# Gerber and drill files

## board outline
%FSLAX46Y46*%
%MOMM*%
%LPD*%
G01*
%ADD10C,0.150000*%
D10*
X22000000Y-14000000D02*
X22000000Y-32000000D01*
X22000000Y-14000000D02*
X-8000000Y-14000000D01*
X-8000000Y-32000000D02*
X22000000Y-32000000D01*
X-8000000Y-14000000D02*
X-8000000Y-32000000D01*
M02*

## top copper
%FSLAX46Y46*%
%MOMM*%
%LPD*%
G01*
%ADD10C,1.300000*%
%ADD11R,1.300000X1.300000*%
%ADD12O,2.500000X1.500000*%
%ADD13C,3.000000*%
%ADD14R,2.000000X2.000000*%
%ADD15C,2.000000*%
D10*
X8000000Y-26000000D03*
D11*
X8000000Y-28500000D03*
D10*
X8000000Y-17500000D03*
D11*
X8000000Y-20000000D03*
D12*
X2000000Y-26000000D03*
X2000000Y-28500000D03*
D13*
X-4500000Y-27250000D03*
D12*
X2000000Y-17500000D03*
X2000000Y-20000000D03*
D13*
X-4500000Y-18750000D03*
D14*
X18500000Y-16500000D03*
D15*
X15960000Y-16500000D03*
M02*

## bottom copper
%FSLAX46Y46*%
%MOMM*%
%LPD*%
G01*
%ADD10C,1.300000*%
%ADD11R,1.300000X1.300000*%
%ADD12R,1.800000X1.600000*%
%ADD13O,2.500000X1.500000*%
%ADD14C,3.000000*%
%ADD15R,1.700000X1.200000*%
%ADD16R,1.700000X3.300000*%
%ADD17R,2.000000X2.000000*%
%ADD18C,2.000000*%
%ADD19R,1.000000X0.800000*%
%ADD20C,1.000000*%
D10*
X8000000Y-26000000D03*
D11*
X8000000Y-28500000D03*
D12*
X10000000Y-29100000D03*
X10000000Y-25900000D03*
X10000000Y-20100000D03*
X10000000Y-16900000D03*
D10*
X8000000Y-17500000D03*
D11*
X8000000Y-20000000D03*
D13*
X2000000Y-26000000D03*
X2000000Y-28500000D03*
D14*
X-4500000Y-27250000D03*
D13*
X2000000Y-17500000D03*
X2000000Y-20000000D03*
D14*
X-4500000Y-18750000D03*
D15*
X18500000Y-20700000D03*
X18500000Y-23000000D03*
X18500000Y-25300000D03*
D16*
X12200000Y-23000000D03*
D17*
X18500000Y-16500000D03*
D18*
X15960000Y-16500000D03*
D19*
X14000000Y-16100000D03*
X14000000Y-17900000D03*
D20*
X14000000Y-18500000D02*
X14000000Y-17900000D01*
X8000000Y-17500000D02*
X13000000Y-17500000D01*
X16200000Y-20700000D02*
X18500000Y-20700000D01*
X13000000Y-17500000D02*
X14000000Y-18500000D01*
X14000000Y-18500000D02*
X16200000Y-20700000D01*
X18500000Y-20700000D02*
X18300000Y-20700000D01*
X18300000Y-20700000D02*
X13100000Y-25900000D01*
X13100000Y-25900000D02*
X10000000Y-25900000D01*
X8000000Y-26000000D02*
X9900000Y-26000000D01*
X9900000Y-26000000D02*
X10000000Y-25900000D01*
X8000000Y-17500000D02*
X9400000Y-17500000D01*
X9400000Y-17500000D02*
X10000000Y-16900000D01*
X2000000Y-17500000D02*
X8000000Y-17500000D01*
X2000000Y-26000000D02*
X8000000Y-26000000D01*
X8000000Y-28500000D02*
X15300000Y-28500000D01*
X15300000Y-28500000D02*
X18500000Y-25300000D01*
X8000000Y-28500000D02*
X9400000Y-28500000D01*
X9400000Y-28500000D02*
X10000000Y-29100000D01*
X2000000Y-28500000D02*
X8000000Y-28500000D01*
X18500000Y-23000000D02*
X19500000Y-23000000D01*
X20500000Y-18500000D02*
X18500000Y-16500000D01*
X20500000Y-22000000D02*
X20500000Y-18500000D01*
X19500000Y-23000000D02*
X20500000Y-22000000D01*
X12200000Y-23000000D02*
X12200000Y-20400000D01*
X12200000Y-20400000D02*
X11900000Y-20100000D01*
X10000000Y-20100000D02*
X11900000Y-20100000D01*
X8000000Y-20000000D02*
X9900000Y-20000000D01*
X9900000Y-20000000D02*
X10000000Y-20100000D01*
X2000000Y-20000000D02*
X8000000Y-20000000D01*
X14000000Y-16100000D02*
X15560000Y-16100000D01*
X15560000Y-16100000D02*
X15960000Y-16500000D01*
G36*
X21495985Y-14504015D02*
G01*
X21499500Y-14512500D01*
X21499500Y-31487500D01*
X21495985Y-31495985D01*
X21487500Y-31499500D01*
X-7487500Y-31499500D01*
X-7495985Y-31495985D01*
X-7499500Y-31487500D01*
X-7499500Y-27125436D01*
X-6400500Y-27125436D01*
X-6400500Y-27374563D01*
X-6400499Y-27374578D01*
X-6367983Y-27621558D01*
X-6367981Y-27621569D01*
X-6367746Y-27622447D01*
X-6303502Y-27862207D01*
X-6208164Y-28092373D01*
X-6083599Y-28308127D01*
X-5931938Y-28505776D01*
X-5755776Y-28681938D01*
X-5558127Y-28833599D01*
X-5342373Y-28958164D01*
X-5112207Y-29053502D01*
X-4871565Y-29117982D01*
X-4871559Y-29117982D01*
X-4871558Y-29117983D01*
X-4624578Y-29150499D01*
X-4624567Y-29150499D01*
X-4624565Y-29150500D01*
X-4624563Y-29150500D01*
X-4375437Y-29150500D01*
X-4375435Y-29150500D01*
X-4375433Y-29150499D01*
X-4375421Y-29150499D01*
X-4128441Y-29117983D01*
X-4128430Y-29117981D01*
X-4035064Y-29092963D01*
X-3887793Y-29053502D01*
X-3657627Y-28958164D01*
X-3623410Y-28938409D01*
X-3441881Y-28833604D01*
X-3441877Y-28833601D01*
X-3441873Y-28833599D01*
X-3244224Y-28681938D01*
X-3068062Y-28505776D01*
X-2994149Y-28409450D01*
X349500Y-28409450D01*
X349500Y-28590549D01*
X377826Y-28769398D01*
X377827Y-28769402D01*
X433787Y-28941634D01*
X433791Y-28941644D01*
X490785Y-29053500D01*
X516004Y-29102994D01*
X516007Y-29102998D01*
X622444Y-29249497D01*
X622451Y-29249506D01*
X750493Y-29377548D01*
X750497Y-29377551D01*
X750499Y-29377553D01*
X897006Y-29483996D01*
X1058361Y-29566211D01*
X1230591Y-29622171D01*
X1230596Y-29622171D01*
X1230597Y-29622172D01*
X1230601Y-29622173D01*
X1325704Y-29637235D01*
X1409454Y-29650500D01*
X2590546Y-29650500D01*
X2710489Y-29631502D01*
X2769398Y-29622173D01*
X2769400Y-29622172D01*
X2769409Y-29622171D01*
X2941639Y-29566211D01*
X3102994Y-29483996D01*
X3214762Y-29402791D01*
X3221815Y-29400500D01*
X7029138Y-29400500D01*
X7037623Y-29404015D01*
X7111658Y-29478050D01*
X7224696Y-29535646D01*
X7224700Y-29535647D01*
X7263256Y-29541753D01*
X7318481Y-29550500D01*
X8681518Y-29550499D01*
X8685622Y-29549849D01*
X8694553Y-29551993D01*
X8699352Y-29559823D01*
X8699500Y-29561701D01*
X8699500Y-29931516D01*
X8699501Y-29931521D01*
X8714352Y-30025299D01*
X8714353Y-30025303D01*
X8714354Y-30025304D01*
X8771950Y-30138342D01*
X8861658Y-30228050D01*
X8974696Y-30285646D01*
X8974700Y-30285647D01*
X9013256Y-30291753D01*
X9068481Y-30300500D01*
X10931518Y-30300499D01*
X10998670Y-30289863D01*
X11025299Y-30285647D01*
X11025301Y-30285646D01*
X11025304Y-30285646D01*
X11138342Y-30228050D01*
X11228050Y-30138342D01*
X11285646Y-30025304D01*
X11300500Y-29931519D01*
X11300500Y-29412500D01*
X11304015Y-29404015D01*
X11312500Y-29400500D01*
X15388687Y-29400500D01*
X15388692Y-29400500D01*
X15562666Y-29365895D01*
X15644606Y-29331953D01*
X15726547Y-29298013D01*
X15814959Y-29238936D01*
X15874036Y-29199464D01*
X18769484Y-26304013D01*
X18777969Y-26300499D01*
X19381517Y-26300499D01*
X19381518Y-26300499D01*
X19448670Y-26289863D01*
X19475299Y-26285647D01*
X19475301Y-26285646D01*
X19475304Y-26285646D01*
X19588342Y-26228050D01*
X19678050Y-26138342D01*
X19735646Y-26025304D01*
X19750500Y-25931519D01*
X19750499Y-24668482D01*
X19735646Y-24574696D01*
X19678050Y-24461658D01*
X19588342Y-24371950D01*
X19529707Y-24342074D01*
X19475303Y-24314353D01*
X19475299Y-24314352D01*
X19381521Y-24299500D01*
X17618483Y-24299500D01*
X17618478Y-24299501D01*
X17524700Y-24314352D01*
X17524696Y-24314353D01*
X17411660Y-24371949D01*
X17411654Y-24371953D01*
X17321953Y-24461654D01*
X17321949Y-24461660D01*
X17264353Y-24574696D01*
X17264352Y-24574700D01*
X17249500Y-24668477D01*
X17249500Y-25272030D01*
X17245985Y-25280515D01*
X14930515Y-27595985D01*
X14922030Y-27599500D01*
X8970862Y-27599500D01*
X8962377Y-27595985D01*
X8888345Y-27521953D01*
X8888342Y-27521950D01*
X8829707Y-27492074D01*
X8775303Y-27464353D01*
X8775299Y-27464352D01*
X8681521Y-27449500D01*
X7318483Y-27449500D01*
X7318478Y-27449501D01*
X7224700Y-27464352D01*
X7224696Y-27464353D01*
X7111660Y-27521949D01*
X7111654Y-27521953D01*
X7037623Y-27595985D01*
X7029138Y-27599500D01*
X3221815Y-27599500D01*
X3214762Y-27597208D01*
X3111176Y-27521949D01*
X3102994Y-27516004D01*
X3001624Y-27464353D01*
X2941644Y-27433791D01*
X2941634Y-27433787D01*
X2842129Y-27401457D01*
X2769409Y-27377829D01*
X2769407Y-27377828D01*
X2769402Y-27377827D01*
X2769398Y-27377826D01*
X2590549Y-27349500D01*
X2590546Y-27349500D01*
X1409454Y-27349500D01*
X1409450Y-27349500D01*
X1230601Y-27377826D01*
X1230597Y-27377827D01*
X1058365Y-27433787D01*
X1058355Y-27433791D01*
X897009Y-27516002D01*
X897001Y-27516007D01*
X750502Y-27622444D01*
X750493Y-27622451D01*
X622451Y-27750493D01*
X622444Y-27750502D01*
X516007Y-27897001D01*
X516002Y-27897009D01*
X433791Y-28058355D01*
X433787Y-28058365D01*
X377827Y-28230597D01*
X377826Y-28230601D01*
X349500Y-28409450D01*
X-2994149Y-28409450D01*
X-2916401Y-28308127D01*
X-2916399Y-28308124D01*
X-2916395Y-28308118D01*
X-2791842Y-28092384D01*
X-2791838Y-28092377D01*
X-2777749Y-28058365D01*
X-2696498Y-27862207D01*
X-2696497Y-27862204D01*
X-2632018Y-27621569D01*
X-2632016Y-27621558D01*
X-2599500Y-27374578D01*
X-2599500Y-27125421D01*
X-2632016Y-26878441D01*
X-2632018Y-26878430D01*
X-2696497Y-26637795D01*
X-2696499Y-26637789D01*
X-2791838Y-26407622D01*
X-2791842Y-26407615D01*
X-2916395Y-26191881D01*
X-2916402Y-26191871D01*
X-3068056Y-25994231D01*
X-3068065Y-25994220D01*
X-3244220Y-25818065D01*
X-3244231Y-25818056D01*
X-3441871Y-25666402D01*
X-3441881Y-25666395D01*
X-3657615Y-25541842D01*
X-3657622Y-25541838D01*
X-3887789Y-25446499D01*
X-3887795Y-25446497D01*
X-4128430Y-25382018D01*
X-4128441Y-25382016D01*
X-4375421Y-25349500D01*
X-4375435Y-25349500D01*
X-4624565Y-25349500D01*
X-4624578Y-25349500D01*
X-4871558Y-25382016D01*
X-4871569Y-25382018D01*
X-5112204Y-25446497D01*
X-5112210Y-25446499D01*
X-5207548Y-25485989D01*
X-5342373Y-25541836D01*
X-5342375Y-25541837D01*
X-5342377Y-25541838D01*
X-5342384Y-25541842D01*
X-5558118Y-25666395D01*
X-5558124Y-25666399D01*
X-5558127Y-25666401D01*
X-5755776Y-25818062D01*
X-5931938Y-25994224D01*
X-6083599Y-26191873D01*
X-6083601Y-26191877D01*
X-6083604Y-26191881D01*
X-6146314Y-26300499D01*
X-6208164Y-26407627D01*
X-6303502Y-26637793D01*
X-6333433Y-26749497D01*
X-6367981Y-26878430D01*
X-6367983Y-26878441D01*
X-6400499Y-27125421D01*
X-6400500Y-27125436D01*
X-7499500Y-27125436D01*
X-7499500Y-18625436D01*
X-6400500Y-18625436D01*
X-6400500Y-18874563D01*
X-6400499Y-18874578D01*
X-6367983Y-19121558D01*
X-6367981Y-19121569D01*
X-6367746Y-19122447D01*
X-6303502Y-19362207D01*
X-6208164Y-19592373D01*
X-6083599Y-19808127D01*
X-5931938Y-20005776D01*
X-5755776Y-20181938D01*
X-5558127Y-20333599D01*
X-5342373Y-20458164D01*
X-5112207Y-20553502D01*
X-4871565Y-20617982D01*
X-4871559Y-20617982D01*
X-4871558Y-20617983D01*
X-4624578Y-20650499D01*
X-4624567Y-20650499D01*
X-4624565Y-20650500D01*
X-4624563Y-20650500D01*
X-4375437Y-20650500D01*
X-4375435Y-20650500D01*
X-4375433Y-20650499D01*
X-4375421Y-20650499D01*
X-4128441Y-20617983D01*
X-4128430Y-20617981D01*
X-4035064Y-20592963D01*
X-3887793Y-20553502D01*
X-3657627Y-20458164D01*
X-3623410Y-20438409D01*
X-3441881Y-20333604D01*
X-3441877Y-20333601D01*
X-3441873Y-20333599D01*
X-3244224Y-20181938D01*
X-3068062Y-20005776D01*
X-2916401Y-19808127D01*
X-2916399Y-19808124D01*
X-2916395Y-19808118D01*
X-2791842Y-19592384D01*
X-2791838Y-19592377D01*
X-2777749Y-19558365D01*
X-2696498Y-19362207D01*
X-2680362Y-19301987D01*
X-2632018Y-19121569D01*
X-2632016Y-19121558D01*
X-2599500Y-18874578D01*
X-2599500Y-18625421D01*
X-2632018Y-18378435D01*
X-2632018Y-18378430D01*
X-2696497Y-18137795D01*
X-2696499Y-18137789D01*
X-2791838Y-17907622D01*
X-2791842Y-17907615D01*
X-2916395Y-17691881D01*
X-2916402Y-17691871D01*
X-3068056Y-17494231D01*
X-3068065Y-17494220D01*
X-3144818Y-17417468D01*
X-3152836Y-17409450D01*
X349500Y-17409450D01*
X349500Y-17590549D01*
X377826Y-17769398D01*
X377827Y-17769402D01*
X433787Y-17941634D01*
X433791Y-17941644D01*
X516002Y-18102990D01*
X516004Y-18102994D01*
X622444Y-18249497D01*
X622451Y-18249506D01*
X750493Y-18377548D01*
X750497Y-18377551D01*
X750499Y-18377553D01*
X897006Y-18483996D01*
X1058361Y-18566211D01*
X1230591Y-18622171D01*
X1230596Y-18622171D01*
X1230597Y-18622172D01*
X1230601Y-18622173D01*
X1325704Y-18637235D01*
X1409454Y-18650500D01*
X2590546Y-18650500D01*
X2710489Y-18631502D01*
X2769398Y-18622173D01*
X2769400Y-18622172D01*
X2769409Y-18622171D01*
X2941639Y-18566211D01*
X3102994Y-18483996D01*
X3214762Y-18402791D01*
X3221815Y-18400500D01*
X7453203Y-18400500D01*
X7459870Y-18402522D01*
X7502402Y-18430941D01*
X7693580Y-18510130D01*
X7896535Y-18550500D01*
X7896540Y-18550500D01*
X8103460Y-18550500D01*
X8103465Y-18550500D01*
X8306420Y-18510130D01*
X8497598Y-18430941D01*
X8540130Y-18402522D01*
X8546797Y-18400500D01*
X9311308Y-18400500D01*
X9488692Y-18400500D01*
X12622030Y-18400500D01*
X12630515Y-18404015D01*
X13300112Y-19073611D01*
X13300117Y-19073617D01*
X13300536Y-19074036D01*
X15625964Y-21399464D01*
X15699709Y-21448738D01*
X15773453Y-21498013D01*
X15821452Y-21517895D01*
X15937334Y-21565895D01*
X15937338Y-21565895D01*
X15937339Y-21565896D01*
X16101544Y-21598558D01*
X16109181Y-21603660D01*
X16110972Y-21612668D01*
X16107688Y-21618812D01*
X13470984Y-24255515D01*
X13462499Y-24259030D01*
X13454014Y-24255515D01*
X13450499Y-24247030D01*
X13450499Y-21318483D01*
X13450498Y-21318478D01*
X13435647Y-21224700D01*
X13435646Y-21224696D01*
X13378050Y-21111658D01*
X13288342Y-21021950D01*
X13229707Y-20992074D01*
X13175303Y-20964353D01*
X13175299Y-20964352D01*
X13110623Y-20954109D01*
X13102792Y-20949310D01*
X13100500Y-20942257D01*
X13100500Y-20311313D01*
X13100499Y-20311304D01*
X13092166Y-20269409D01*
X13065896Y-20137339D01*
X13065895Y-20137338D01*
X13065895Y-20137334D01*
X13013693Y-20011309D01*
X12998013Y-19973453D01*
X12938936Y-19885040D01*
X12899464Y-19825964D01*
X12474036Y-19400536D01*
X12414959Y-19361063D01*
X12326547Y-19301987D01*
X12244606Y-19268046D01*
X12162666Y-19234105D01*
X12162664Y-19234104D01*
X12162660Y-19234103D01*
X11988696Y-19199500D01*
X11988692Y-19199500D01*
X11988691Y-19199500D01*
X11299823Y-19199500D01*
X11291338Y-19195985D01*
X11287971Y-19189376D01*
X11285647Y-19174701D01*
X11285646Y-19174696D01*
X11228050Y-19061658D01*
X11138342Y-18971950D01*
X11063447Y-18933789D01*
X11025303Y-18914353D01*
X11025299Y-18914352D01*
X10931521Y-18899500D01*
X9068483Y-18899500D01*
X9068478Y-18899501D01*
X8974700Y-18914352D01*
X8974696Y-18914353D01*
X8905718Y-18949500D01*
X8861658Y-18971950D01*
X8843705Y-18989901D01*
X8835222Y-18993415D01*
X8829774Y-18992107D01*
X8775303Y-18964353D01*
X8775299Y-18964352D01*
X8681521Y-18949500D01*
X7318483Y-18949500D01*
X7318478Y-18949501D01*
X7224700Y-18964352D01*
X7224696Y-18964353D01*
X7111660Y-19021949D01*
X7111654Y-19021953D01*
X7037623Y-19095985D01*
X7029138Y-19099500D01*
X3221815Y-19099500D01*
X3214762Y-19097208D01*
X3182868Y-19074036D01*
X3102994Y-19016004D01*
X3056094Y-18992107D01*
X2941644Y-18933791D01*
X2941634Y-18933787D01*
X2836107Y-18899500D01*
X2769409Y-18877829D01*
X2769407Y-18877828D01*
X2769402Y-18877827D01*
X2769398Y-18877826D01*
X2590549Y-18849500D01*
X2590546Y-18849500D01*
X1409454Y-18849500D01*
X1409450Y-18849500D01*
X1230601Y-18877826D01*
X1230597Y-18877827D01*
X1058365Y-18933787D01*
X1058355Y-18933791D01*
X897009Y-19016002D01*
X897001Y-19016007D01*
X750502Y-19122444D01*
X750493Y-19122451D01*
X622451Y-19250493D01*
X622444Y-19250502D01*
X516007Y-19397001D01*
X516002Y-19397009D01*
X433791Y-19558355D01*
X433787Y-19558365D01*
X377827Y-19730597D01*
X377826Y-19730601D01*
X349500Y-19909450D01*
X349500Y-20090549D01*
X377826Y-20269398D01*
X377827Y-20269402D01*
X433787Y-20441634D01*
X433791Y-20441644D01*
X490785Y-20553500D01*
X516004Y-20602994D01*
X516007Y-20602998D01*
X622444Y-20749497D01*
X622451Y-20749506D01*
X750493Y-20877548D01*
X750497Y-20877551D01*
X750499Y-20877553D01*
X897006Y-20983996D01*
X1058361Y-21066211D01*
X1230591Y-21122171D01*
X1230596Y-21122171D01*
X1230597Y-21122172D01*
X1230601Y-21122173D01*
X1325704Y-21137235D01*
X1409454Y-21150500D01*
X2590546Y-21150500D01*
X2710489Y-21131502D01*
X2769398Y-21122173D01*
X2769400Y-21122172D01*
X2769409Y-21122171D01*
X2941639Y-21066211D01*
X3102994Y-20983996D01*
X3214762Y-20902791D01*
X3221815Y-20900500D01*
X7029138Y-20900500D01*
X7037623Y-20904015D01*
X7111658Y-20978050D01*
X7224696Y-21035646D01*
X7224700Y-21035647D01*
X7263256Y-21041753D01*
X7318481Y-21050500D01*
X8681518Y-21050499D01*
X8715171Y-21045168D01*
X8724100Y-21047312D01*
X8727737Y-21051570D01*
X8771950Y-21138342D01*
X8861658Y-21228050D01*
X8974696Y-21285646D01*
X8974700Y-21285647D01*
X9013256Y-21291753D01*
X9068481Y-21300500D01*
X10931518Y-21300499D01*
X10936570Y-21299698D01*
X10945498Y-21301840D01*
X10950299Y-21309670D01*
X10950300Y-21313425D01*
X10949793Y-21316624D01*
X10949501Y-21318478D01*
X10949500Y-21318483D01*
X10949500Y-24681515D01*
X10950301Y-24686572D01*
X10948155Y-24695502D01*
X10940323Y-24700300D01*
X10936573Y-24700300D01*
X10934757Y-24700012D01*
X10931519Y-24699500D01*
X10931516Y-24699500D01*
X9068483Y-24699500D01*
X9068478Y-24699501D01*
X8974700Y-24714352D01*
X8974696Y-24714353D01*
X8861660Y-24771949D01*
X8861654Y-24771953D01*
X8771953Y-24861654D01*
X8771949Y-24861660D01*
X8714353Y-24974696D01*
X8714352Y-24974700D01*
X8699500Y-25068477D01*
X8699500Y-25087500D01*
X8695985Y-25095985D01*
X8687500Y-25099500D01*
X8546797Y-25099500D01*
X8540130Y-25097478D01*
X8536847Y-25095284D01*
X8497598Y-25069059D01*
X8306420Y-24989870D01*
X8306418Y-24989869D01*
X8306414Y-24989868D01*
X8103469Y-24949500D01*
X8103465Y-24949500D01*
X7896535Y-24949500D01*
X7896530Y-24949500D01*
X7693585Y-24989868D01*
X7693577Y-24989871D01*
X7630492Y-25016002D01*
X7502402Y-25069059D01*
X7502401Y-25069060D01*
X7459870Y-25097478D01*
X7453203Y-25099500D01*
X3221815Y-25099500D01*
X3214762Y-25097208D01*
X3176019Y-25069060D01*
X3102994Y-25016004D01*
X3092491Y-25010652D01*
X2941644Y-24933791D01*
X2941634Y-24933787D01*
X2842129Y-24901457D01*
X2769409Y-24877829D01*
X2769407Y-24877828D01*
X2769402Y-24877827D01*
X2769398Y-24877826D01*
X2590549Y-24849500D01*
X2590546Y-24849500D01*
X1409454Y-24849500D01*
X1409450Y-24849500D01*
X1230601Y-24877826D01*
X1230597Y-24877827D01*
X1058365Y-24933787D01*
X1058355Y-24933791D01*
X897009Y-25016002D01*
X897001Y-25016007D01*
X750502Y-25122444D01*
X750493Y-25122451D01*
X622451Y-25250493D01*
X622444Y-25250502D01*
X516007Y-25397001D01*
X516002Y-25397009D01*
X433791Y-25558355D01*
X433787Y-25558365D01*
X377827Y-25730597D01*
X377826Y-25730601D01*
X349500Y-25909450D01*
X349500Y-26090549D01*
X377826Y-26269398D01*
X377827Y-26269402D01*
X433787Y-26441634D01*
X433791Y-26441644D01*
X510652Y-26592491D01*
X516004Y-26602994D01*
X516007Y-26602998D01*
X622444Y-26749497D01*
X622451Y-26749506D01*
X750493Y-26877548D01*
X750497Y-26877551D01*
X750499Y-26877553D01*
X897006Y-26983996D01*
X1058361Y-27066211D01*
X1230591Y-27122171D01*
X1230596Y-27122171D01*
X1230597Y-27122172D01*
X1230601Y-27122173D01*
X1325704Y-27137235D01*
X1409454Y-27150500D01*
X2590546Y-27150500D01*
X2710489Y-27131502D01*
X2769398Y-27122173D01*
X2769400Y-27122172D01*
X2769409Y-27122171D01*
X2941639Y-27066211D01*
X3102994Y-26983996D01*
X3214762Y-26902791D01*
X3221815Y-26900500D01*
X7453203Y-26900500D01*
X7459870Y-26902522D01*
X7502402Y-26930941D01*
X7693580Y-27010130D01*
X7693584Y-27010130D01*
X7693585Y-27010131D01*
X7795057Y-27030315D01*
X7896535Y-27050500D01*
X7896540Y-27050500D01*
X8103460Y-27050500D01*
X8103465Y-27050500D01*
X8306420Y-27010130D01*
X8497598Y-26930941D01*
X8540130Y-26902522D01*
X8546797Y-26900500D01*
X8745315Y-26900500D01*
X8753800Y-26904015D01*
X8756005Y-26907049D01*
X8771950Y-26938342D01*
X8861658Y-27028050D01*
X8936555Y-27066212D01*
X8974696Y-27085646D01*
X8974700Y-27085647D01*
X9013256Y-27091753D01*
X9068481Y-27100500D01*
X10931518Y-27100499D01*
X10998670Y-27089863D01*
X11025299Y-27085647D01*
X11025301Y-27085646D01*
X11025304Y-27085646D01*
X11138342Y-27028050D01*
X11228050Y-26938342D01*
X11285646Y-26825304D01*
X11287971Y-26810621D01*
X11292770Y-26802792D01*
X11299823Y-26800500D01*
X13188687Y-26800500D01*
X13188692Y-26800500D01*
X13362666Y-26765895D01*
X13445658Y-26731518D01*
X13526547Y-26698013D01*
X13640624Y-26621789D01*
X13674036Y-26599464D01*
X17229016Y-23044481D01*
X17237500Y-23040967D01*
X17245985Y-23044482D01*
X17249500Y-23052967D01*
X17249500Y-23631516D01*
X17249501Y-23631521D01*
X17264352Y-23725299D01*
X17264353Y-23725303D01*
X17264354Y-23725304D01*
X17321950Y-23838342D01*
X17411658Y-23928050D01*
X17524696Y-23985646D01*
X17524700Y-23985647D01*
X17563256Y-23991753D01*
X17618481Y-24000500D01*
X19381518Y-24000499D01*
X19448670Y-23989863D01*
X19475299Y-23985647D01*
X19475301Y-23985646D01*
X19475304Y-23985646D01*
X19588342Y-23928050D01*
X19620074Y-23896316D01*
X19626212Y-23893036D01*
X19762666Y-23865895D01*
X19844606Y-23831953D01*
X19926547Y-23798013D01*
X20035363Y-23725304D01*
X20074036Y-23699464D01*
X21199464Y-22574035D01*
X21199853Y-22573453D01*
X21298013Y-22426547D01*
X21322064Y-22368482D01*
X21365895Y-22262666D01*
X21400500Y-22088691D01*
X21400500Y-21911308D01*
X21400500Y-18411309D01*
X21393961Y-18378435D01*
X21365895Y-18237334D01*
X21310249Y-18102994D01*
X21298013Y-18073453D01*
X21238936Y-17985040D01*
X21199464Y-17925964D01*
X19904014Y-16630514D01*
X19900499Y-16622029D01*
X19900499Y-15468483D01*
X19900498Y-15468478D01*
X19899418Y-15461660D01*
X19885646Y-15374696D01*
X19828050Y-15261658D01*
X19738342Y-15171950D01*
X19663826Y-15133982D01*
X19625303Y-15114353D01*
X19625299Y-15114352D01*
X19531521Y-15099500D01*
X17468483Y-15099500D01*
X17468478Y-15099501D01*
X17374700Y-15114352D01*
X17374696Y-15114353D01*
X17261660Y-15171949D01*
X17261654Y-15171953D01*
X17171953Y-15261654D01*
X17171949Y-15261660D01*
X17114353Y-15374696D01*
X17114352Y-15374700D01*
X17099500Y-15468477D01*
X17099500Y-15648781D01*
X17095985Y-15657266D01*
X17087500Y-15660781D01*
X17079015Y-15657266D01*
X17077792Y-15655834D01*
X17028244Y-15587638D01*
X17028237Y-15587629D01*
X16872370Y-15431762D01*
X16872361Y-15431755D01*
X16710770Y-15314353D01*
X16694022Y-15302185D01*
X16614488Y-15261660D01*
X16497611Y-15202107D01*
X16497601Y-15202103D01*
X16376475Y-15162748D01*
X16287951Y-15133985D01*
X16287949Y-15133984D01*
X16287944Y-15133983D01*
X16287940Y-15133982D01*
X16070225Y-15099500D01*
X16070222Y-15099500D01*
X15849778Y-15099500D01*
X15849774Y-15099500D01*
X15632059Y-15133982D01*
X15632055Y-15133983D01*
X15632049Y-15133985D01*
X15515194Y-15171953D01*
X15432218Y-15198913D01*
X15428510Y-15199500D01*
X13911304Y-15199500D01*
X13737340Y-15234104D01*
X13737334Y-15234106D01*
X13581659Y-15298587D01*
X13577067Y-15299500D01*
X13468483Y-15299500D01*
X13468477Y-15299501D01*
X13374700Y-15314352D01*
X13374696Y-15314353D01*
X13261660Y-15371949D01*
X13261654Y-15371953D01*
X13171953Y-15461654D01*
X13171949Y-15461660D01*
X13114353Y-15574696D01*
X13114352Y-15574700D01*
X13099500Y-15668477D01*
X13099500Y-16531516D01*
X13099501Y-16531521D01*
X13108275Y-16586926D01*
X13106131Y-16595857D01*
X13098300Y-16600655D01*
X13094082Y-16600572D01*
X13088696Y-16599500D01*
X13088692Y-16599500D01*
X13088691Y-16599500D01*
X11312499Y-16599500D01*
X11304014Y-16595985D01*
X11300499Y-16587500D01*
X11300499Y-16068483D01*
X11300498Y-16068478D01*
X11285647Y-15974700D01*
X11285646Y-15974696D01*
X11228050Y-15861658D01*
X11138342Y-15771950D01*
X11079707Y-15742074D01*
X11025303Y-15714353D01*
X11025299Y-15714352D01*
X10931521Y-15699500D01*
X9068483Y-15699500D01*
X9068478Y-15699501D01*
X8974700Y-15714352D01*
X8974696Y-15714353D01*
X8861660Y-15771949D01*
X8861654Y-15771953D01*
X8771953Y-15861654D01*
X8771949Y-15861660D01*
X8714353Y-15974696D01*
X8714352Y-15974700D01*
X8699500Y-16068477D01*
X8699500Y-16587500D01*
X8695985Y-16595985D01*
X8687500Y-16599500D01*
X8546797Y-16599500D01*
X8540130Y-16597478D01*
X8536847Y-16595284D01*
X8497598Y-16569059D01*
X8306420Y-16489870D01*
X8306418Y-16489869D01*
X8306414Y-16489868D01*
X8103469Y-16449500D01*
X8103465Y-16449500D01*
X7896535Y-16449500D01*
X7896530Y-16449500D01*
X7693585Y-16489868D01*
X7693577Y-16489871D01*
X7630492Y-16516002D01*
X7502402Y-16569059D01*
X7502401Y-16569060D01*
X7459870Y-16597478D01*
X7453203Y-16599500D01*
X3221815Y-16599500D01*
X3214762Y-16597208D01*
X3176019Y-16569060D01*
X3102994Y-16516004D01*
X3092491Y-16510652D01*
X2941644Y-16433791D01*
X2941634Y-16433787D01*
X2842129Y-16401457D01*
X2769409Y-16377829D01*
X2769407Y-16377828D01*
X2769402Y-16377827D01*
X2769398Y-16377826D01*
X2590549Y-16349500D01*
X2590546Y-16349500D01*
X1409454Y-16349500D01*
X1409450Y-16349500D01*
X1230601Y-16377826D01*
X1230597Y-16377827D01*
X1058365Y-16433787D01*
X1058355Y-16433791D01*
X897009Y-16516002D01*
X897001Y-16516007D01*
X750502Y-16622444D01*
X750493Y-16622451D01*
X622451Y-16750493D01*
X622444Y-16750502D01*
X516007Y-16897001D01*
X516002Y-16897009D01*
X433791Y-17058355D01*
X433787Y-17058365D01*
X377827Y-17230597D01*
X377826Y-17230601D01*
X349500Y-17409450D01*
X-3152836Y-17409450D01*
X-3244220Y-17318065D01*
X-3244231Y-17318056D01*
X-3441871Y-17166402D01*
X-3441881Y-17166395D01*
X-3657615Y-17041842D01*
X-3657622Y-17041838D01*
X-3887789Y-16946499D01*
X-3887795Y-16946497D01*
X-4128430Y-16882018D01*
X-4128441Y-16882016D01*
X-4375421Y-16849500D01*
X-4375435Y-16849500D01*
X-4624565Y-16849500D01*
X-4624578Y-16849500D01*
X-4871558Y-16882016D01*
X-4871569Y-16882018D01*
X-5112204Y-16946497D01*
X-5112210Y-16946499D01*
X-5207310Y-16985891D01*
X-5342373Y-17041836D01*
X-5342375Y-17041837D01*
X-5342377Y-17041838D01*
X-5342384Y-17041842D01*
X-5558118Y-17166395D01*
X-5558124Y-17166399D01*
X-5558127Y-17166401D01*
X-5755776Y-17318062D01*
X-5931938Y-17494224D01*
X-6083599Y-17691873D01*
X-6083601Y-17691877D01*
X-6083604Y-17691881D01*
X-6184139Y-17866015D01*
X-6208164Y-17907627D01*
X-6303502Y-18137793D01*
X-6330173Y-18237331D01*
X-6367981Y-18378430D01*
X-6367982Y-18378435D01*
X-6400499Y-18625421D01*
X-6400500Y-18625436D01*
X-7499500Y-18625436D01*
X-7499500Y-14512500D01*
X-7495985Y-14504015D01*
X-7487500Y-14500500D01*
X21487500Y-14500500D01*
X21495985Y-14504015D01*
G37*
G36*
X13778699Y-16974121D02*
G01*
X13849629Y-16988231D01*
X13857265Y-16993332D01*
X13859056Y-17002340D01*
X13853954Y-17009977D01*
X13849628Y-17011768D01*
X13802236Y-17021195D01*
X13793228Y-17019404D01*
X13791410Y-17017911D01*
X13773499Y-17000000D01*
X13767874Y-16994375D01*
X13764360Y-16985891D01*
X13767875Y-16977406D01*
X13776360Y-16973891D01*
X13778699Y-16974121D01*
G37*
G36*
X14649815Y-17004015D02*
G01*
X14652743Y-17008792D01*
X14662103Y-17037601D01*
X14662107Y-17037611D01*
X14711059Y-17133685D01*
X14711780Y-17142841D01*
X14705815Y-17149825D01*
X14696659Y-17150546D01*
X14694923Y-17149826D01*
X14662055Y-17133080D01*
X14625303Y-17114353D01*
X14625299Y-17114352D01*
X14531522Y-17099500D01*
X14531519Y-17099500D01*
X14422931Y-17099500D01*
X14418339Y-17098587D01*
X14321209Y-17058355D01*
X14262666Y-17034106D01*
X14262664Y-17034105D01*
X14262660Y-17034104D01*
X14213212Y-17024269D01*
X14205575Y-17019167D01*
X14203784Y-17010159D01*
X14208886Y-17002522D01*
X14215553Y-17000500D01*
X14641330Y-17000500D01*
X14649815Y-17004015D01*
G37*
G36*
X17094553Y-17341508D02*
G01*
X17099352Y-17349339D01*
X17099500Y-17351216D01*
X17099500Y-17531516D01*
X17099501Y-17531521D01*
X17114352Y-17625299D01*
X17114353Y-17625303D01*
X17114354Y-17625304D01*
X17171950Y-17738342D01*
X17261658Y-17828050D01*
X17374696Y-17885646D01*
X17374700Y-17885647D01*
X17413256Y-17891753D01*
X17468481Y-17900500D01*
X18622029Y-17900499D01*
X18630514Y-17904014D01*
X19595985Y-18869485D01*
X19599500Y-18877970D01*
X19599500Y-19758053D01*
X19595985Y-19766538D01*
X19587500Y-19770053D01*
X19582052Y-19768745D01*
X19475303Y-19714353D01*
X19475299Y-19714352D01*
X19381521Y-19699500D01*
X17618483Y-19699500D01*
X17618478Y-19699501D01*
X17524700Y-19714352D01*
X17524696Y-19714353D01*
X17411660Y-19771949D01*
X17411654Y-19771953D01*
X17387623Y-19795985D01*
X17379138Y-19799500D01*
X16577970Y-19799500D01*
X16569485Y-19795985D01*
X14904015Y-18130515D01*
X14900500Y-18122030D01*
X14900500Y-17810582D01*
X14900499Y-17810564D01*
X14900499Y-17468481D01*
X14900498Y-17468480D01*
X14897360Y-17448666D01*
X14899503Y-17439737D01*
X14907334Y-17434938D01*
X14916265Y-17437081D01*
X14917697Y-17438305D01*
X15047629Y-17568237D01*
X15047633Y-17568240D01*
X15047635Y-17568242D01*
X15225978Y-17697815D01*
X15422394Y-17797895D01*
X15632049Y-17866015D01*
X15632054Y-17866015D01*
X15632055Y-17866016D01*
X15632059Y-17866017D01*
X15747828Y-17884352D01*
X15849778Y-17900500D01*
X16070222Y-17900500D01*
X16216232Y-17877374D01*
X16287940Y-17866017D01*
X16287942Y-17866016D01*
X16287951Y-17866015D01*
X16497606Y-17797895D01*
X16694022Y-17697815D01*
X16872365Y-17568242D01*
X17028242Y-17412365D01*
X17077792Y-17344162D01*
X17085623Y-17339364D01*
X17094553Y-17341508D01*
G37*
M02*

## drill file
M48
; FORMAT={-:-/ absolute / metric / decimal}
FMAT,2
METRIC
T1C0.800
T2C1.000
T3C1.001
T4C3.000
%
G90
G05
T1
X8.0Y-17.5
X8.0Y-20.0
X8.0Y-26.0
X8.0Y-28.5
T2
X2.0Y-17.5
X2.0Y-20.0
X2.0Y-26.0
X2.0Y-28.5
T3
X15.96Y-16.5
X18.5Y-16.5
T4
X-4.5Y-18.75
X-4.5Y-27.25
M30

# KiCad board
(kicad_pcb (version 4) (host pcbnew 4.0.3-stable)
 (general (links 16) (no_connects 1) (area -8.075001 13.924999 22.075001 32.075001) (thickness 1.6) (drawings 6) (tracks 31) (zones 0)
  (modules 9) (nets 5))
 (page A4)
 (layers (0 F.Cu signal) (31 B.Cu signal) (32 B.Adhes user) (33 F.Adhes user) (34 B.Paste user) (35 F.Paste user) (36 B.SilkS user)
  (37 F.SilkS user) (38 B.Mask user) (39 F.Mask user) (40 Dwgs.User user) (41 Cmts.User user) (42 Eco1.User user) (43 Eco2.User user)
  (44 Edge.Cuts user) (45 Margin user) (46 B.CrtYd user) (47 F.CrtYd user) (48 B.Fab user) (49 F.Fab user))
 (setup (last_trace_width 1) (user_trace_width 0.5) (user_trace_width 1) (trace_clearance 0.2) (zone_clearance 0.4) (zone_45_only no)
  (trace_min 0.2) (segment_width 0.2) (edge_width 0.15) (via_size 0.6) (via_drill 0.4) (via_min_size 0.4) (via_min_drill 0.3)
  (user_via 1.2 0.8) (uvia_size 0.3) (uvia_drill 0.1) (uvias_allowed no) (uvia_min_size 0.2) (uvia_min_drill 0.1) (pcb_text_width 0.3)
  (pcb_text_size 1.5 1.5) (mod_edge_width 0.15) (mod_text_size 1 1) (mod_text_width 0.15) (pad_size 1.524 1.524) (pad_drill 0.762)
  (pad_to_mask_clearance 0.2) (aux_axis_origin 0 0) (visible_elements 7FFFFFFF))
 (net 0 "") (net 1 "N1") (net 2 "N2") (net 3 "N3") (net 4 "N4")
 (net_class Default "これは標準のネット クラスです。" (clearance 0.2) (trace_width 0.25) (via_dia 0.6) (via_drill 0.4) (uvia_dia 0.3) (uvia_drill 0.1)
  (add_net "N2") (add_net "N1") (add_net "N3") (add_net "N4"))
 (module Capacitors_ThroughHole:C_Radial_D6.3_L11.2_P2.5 (layer F.Cu) (at 8 28.5 90)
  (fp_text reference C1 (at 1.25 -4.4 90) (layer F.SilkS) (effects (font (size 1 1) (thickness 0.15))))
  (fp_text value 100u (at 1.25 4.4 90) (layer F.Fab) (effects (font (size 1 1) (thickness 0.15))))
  (pad 2 thru_hole circle (at 2.5 0 90) (size 1.3 1.3) (drill 0.8) (layers *.Cu *.Mask F.SilkS) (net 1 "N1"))
  (pad 1 thru_hole rect (at 0 0 90) (size 1.3 1.3) (drill 0.8) (layers *.Cu *.Mask F.SilkS) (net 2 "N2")))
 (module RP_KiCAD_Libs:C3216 (layer B.Cu) (at 10 27.5 90)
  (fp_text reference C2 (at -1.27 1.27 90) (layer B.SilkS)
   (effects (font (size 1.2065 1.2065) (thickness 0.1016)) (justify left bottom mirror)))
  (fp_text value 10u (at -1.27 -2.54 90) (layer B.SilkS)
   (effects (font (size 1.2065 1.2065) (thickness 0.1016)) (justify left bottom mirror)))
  (pad 1 smd rect (at -1.6 0 90) (size 1.6 1.8) (layers B.Cu B.Paste B.Mask) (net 2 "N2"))
  (pad 2 smd rect (at 1.6 0 90) (size 1.6 1.8) (layers B.Cu B.Paste B.Mask) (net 1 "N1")))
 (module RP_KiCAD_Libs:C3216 (layer B.Cu) (at 10 18.5 90)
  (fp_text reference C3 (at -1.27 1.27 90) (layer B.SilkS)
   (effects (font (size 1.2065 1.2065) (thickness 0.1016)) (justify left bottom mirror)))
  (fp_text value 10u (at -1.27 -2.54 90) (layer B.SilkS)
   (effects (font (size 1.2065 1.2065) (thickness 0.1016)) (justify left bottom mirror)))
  (pad 1 smd rect (at -1.6 0 90) (size 1.6 1.8) (layers B.Cu B.Paste B.Mask) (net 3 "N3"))
  (pad 2 smd rect (at 1.6 0 90) (size 1.6 1.8) (layers B.Cu B.Paste B.Mask) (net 1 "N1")))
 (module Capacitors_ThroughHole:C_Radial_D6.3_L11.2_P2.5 (layer F.Cu) (at 8 20 90)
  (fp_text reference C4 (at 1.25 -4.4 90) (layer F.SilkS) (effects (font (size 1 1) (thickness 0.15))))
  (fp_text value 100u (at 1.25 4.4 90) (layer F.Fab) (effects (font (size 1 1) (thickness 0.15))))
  (pad 2 thru_hole circle (at 2.5 0 90) (size 1.3 1.3) (drill 0.8) (layers *.Cu *.Mask F.SilkS) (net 1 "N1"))
  (pad 1 thru_hole rect (at 0 0 90) (size 1.3 1.3) (drill 0.8) (layers *.Cu *.Mask F.SilkS) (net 3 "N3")))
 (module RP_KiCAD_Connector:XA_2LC (layer F.Cu) (at 2 26 270)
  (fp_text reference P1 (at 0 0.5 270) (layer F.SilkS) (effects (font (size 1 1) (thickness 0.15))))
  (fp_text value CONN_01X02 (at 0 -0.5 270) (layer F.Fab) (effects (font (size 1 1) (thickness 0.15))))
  (pad 1 thru_hole oval (at 0 0 270) (size 1.5 2.5) (drill 1) (layers *.Cu *.Mask F.SilkS) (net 1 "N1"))
  (pad 2 thru_hole oval (at 2.5 0 270) (size 1.5 2.5) (drill 1) (layers *.Cu *.Mask F.SilkS) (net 2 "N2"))
  (pad "" thru_hole circle (at 1.25 6.5 270) (size 3 3) (drill 3) (layers *.Cu *.Mask F.SilkS) (clearance -0.3)))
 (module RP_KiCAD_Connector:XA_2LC (layer F.Cu) (at 2 17.5 270)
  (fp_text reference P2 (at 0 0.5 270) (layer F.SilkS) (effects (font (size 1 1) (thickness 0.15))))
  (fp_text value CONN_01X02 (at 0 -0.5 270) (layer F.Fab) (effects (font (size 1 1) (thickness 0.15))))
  (pad 1 thru_hole oval (at 0 0 270) (size 1.5 2.5) (drill 1) (layers *.Cu *.Mask F.SilkS) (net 1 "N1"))
  (pad 2 thru_hole oval (at 2.5 0 270) (size 1.5 2.5) (drill 1) (layers *.Cu *.Mask F.SilkS) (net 3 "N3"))
  (pad "" thru_hole circle (at 1.25 6.5 270) (size 3 3) (drill 3) (layers *.Cu *.Mask F.SilkS) (clearance -0.3)))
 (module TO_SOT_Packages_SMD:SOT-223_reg (layer B.Cu) (at 18.5 23 270)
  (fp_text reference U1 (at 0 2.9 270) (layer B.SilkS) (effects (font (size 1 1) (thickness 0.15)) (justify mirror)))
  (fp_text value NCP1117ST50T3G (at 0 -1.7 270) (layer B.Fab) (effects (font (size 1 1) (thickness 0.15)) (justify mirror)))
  (pad 1 smd rect (at -2.3 0 270) (size 1.2 1.7) (layers B.Cu B.Paste B.Mask) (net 1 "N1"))
  (pad 2 smd rect (at 0 0 270) (size 1.2 1.7) (layers B.Cu B.Paste B.Mask) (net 3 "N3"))
  (pad 3 smd rect (at 2.3 0 270) (size 1.2 1.7) (layers B.Cu B.Paste B.Mask) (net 2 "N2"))
  (pad 2 smd rect (at 0 6.3 270) (size 3.3 1.7) (layers B.Cu B.Paste B.Mask) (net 3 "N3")))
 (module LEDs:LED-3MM (layer F.Cu) (at 18.5 16.5 180)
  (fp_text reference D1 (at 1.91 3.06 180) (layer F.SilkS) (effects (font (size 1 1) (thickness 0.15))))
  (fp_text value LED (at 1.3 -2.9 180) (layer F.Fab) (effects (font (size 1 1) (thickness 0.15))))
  (pad 1 thru_hole rect (at 0 0 270) (size 2 2) (drill 1.00076) (layers *.Cu *.Mask F.SilkS) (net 3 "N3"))
  (pad 2 thru_hole circle (at 2.54 0 180) (size 2 2) (drill 1.00076) (layers *.Cu *.Mask F.SilkS) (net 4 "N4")))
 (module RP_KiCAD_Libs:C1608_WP (layer B.Cu) (at 14 17 270)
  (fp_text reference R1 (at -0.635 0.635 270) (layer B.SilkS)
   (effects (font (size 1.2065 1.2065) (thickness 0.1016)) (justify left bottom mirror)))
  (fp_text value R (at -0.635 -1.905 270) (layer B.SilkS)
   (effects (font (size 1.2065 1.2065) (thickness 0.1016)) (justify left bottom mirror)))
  (pad 1 smd rect (at -0.9 0 270) (size 0.8 1) (layers B.Cu B.Paste B.Mask) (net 4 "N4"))
  (pad 2 smd rect (at 0.9 0 270) (size 0.8 1) (layers B.Cu B.Paste B.Mask) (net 1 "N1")))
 (gr_line (start 22 14) (end 22 32) (angle 90) (layer Edge.Cuts) (width 0.15))
 (gr_line (start 22 14) (end -8 14) (angle 90) (layer Edge.Cuts) (width 0.15))
 (gr_line (start -8 32) (end 22 32) (angle 90) (layer Edge.Cuts) (width 0.15))
 (gr_line (start -8 14) (end -8 32) (angle 90) (layer Edge.Cuts) (width 0.15))
 (segment (start 14 18.5) (end 14 17.9) (width 1) (layer B.Cu) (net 1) (status 800000))
 (segment (start 8 17.5) (end 13 17.5) (width 1) (layer B.Cu) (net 1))
 (segment (start 16.2 20.7) (end 18.5 20.7) (width 1) (layer B.Cu) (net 1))
 (segment (start 13 17.5) (end 14 18.5) (width 1) (layer B.Cu) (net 1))
 (segment (start 14 18.5) (end 16.2 20.7) (width 1) (layer B.Cu) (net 1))
 (segment (start 18.5 20.7) (end 18.3 20.7) (width 1) (layer B.Cu) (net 1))
 (segment (start 18.3 20.7) (end 13.1 25.9) (width 1) (layer B.Cu) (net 1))
 (segment (start 13.1 25.9) (end 10 25.9) (width 1) (layer B.Cu) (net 1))
 (segment (start 8 26) (end 9.9 26) (width 1) (layer B.Cu) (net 1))
 (segment (start 9.9 26) (end 10 25.9) (width 1) (layer B.Cu) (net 1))
 (segment (start 8 17.5) (end 9.4 17.5) (width 1) (layer B.Cu) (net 1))
 (segment (start 9.4 17.5) (end 10 16.9) (width 1) (layer B.Cu) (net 1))
 (segment (start 2 17.5) (end 8 17.5) (width 1) (layer B.Cu) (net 1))
 (segment (start 2 26) (end 8 26) (width 1) (layer B.Cu) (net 1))
 (segment (start 8 28.5) (end 15.3 28.5) (width 1) (layer B.Cu) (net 2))
 (segment (start 15.3 28.5) (end 18.5 25.3) (width 1) (layer B.Cu) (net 2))
 (segment (start 8 28.5) (end 9.4 28.5) (width 1) (layer B.Cu) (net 2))
 (segment (start 9.4 28.5) (end 10 29.1) (width 1) (layer B.Cu) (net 2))
 (segment (start 2 28.5) (end 8 28.5) (width 1) (layer B.Cu) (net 2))
 (segment (start 18.5 23) (end 19.5 23) (width 1) (layer B.Cu) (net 3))
 (segment (start 20.5 18.5) (end 18.5 16.5) (width 1) (layer B.Cu) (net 3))
 (segment (start 20.5 22) (end 20.5 18.5) (width 1) (layer B.Cu) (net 3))
 (segment (start 19.5 23) (end 20.5 22) (width 1) (layer B.Cu) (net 3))
 (segment (start 12.2 23) (end 12.2 20.4) (width 1) (layer B.Cu) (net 3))
 (segment (start 12.2 20.4) (end 11.9 20.1) (width 1) (layer B.Cu) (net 3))
 (segment (start 10 20.1) (end 11.9 20.1) (width 1) (layer B.Cu) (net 3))
 (segment (start 8 20) (end 9.9 20) (width 1) (layer B.Cu) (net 3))
 (segment (start 9.9 20) (end 10 20.1) (width 1) (layer B.Cu) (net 3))
 (segment (start 2 20) (end 8 20) (width 1) (layer B.Cu) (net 3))
 (segment (start 14 16.1) (end 15.56 16.1) (width 1) (layer B.Cu) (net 4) (status C00000))
 (segment (start 15.56 16.1) (end 15.96 16.5) (width 1) (layer B.Cu) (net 4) (status C00000))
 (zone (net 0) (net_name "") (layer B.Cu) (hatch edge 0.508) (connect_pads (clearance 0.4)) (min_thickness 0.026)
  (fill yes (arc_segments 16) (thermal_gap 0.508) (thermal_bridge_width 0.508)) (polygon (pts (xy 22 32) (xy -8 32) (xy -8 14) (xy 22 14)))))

